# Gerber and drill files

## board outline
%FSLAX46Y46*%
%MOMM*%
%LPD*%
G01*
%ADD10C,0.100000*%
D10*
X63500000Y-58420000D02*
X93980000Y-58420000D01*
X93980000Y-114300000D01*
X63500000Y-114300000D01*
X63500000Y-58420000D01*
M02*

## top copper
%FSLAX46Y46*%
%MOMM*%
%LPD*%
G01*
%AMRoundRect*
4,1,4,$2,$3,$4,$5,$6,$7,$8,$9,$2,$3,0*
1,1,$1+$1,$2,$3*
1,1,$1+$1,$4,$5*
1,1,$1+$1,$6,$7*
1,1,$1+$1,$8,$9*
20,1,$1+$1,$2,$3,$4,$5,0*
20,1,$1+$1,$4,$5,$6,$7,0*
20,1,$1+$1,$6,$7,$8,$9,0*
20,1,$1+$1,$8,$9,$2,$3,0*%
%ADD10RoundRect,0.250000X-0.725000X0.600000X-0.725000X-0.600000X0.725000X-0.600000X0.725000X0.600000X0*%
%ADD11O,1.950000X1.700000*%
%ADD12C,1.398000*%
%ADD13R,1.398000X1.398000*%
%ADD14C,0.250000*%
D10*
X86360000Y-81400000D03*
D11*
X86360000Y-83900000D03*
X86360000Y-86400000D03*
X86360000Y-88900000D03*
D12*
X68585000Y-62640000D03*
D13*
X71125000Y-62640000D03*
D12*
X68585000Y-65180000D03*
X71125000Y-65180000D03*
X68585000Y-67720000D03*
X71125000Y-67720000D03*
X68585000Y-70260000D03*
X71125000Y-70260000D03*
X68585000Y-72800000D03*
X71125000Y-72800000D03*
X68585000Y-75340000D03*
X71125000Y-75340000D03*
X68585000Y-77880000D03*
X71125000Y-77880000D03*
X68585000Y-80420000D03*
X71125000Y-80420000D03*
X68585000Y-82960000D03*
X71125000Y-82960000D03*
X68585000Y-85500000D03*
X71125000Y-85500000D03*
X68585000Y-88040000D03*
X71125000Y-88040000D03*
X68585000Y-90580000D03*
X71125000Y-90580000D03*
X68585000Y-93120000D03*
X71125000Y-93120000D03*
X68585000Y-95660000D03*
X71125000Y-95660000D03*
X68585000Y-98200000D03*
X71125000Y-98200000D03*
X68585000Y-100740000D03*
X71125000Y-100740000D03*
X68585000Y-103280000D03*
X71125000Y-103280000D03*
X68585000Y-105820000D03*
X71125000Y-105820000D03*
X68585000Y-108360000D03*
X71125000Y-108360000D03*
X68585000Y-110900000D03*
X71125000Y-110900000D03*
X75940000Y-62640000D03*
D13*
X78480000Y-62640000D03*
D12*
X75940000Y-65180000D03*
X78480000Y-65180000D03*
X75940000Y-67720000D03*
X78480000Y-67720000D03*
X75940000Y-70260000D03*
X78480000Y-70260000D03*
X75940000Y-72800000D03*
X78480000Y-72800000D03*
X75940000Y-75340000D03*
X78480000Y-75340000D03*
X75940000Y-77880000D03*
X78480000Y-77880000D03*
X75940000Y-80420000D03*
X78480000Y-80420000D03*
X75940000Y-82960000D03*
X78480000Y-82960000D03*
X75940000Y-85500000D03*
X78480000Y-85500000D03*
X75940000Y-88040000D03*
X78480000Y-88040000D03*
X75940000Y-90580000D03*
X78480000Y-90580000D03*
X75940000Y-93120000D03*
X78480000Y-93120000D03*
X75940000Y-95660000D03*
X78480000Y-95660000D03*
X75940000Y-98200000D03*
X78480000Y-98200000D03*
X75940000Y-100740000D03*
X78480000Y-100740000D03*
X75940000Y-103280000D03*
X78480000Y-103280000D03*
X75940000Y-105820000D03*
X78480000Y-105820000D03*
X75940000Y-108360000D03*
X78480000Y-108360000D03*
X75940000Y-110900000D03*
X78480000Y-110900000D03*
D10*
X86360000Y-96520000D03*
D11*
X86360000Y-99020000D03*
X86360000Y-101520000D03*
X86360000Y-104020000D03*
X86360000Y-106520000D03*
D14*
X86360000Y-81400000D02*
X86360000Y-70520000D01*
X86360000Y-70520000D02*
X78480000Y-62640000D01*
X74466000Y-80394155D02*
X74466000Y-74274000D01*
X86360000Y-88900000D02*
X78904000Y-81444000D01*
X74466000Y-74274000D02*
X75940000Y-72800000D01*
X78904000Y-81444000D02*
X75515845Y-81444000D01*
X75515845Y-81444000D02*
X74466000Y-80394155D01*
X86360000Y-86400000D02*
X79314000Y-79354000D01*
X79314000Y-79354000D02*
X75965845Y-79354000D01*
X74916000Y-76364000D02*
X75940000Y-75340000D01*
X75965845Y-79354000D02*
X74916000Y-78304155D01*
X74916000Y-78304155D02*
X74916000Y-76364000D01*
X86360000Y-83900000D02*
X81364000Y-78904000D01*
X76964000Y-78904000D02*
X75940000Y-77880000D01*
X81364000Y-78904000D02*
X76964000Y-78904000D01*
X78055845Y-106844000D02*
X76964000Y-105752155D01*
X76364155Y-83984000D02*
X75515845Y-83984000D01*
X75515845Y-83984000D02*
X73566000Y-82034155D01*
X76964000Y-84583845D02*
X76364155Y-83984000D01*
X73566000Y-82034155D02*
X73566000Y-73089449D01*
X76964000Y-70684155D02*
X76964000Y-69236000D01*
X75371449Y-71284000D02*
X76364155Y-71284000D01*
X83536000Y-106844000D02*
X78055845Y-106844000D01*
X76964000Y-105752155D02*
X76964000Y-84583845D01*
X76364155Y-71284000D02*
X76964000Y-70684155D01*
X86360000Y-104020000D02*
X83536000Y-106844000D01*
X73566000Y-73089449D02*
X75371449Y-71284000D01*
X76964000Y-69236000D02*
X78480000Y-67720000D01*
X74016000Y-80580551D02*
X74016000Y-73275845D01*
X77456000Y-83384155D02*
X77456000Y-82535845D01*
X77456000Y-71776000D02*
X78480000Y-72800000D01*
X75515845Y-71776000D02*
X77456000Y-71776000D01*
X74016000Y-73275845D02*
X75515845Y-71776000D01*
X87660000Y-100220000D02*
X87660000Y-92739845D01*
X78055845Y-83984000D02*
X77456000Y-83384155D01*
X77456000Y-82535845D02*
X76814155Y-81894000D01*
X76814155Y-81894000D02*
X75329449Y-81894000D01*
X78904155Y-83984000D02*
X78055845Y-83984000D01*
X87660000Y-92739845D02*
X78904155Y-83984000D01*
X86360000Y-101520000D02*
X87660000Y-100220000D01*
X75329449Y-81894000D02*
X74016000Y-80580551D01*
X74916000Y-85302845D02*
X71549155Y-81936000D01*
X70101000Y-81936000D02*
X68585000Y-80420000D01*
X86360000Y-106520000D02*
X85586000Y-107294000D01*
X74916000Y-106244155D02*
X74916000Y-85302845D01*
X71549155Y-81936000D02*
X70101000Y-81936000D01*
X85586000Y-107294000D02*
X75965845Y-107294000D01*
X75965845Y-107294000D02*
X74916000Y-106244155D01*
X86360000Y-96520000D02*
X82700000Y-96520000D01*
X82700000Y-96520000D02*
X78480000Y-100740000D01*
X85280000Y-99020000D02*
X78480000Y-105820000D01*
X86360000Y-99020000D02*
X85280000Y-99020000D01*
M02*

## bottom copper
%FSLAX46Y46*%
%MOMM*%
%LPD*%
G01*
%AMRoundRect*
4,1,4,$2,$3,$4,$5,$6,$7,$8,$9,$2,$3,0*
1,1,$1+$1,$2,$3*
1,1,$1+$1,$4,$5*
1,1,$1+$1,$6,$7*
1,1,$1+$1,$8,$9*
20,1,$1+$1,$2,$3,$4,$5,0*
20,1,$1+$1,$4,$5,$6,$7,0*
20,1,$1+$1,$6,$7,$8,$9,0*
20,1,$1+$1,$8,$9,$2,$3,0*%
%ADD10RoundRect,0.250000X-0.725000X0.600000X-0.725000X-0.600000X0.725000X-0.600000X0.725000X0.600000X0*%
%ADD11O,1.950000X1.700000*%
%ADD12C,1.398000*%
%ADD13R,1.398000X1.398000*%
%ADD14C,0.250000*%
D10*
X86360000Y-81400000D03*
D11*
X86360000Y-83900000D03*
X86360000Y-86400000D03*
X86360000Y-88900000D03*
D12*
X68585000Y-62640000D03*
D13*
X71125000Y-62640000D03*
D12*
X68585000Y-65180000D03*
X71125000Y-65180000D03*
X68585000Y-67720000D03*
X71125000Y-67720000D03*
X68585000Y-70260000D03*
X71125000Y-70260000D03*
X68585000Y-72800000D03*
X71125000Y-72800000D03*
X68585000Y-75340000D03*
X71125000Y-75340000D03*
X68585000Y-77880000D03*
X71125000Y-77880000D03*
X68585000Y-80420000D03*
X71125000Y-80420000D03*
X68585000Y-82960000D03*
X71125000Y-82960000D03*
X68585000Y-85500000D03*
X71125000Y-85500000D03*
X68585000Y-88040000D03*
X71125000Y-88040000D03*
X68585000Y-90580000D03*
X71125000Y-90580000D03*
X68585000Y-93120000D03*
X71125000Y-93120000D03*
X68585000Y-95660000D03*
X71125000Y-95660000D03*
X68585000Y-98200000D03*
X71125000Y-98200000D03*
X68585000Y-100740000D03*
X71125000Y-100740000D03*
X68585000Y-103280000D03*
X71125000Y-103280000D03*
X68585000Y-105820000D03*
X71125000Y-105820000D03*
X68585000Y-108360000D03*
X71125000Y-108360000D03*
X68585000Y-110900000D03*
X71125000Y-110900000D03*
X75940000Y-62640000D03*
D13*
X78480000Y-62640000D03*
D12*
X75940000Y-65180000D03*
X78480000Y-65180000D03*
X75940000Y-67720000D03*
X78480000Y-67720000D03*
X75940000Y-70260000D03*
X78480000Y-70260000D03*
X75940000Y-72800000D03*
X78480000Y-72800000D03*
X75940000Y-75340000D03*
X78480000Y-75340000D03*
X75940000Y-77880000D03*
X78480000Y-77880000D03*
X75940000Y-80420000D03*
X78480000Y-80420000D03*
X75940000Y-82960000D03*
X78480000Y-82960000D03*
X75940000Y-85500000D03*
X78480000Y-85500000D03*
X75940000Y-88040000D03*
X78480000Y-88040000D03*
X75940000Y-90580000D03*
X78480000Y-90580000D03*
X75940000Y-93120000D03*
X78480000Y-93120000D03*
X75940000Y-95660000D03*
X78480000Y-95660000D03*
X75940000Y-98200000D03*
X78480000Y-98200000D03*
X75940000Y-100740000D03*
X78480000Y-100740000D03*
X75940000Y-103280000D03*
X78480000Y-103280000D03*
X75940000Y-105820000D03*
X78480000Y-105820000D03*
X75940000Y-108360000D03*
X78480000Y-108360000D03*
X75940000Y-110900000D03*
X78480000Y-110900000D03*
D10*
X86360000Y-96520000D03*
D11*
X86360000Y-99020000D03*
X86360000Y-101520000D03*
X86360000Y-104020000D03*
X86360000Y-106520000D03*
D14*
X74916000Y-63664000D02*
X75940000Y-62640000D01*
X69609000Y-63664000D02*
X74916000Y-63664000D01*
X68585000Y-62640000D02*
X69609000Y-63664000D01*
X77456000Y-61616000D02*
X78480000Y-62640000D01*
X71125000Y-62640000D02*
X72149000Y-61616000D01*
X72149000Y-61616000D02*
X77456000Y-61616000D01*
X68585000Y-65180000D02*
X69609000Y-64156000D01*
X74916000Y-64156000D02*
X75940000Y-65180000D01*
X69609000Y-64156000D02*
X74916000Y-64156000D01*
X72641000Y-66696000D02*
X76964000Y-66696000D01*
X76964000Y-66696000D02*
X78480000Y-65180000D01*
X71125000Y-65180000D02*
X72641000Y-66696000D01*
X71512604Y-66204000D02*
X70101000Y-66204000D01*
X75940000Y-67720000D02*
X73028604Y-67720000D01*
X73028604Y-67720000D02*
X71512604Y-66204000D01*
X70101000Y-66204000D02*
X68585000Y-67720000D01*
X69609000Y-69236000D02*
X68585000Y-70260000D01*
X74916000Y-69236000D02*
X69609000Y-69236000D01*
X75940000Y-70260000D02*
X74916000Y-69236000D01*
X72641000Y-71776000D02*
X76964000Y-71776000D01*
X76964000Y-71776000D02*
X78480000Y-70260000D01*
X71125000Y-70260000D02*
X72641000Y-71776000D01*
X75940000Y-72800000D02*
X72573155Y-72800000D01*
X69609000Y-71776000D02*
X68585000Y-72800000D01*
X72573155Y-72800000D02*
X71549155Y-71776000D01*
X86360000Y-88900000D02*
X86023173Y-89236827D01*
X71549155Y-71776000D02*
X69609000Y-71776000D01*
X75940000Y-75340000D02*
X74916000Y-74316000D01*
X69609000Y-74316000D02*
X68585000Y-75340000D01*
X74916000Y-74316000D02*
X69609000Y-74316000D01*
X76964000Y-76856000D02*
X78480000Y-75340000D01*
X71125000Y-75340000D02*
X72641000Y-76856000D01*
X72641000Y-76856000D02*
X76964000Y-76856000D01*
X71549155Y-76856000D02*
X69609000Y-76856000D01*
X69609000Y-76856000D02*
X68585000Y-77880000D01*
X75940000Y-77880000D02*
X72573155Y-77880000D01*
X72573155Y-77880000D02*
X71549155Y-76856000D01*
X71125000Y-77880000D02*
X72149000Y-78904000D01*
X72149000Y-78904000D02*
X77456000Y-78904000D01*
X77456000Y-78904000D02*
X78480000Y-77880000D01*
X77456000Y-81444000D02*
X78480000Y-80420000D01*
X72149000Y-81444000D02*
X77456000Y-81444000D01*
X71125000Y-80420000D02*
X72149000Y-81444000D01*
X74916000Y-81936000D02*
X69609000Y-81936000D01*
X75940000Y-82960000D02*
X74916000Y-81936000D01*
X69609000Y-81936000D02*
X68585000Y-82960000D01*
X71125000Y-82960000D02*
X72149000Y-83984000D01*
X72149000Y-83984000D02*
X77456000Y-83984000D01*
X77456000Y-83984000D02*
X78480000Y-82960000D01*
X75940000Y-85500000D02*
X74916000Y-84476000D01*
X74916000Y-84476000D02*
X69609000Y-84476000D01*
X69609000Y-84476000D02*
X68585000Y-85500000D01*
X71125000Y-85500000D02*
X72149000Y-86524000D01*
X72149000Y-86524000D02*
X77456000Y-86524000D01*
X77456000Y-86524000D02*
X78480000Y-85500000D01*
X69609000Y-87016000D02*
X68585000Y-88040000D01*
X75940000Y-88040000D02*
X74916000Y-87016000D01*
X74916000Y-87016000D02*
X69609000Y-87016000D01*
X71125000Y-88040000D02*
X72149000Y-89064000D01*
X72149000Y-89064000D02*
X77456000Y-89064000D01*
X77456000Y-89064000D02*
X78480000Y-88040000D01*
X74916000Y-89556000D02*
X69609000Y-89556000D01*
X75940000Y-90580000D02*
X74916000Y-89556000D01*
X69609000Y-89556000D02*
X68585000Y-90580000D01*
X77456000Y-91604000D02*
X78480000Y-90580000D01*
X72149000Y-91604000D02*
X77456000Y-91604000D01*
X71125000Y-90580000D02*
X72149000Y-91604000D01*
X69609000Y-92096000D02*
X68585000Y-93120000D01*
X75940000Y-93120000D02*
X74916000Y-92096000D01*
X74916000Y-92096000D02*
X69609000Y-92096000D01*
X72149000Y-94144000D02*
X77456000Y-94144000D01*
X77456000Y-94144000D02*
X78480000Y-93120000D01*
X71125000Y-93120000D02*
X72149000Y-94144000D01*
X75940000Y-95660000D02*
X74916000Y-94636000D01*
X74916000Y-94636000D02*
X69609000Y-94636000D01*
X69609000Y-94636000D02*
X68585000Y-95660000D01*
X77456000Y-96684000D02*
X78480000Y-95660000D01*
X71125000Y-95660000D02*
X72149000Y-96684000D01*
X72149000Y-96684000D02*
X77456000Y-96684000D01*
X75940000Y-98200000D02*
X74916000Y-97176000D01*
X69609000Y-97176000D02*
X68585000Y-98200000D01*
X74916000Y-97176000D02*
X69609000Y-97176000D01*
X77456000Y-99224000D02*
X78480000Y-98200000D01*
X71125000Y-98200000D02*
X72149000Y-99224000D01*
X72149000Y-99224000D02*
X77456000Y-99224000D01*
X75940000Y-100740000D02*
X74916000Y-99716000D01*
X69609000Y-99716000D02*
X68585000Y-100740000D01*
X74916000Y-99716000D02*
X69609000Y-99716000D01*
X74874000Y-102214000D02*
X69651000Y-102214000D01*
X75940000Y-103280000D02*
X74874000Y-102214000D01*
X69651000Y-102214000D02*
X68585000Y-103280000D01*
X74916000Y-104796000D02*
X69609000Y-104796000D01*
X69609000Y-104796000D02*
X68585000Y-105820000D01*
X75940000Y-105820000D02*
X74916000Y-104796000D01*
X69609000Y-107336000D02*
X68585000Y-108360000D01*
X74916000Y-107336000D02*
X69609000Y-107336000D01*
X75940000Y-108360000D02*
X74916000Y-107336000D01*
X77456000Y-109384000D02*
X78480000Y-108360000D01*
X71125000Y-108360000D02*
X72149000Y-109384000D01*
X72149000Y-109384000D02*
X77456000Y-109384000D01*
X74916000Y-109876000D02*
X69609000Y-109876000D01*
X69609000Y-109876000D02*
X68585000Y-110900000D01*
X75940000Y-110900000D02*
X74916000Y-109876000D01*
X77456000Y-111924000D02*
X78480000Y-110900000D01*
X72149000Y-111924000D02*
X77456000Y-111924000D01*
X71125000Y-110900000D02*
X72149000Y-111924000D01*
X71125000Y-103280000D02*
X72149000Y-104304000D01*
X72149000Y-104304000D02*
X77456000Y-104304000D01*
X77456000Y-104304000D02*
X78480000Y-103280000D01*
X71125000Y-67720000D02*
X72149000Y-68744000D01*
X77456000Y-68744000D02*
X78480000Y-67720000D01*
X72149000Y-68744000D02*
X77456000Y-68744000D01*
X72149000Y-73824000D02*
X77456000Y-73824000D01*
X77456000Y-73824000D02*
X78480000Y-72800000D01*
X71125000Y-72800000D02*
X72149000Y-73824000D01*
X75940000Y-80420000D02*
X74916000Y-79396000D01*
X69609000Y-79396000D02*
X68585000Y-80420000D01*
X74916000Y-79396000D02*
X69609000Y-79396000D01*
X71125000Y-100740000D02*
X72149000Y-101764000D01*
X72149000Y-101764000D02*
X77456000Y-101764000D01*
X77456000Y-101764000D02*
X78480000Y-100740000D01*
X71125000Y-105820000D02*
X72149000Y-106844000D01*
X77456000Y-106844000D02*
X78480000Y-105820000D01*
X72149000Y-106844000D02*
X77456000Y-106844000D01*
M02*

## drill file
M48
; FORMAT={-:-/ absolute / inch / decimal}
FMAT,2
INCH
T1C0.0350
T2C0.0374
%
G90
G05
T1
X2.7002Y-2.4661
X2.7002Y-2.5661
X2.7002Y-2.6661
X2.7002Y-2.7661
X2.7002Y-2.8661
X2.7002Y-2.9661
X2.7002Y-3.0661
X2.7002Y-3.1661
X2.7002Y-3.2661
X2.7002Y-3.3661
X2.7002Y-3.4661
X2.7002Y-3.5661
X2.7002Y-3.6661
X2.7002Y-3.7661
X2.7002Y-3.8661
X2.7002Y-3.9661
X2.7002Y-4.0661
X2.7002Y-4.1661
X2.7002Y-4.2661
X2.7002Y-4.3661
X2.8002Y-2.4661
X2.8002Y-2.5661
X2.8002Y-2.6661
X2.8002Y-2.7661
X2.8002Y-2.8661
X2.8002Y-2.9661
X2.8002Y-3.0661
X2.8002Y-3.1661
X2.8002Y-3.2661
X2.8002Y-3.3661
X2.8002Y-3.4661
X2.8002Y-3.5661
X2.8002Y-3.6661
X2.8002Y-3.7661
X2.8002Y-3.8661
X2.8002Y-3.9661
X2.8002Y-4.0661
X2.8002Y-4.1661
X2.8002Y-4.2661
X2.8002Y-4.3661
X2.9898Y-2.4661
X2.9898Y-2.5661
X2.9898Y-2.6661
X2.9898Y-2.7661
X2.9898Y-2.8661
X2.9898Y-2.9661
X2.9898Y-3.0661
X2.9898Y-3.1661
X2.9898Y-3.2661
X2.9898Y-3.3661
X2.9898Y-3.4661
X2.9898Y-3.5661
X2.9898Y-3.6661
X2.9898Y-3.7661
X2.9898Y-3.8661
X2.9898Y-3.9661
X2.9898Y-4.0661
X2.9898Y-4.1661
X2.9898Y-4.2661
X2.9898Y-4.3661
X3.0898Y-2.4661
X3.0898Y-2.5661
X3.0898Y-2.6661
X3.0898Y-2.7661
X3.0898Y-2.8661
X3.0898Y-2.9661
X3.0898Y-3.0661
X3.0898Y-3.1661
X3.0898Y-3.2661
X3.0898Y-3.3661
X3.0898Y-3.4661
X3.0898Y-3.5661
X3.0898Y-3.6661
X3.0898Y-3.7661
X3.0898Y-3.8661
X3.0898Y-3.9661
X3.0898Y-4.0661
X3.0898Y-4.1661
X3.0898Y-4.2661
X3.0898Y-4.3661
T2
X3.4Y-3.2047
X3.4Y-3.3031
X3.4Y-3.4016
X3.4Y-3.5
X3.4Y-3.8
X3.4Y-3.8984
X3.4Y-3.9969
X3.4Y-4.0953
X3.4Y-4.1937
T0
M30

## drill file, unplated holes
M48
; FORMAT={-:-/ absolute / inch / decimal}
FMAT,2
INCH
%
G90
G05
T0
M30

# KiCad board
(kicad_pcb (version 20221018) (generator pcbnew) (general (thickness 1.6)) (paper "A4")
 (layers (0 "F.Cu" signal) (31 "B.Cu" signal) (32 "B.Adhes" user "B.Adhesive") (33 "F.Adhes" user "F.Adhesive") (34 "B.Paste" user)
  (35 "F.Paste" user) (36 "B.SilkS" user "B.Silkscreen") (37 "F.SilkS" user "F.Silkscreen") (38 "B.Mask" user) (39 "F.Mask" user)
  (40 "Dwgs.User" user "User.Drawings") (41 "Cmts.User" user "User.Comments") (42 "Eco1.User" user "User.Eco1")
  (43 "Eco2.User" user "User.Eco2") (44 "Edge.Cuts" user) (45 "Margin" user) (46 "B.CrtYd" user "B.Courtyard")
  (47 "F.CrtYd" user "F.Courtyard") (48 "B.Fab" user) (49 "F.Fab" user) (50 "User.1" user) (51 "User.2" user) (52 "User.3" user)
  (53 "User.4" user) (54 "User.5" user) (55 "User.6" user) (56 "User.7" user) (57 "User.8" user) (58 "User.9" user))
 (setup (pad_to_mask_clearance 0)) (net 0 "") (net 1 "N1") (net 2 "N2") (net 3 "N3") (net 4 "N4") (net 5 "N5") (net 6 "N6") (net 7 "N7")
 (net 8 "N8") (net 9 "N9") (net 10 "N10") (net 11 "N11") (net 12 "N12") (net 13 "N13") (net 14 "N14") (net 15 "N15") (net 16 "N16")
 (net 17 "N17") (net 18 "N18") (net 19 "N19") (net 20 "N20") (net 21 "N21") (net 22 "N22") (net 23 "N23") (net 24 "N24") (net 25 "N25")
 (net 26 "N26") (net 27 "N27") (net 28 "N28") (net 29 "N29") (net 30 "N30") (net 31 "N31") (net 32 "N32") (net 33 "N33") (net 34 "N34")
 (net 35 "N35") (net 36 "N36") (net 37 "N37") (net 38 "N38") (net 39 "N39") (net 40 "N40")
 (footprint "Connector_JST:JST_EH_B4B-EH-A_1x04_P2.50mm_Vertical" (layer "F.Cu") (at 86.36 81.4 -90)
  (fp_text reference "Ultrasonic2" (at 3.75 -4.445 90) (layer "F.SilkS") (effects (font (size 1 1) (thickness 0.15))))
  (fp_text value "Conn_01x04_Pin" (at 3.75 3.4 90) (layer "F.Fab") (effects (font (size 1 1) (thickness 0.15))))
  (pad "1" thru_hole roundrect (at 0 0 270) (size 1.7 1.95) (drill 0.95) (layers "*.Cu" "*.Mask") (roundrect_rratio 0.1470588235)
   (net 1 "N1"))
  (pad "2" thru_hole oval (at 2.5 0 270) (size 1.7 1.95) (drill 0.95) (layers "*.Cu" "*.Mask") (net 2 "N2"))
  (pad "3" thru_hole oval (at 5 0 270) (size 1.7 1.95) (drill 0.95) (layers "*.Cu" "*.Mask") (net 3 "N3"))
  (pad "4" thru_hole oval (at 7.5 0 270) (size 1.7 1.95) (drill 0.95) (layers "*.Cu" "*.Mask") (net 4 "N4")))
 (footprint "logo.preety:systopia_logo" (layer "F.Cu") (at 87.63 68.58)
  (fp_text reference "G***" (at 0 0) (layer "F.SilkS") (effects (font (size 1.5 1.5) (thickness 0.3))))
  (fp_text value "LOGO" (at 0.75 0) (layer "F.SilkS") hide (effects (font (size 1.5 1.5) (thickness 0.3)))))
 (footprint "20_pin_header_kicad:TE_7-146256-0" (layer "F.Cu") (at 69.855 86.77 -90)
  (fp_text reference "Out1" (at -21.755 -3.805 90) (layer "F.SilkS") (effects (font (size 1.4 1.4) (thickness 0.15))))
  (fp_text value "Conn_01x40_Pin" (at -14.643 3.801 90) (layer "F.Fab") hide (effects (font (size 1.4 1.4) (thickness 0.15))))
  (pad "1" thru_hole circle (at -24.13 1.27 270) (size 1.398 1.398) (drill 0.89) (layers "*.Cu" "*.Mask") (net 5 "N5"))
  (pad "2" thru_hole rect (at -24.13 -1.27 270) (size 1.398 1.398) (drill 0.89) (layers "*.Cu" "*.Mask") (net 1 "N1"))
  (pad "3" thru_hole circle (at -21.59 1.27 270) (size 1.398 1.398) (drill 0.89) (layers "*.Cu" "*.Mask") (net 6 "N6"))
  (pad "4" thru_hole circle (at -21.59 -1.27 270) (size 1.398 1.398) (drill 0.89) (layers "*.Cu" "*.Mask") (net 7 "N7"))
  (pad "5" thru_hole circle (at -19.05 1.27 270) (size 1.398 1.398) (drill 0.89) (layers "*.Cu" "*.Mask") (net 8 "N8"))
  (pad "6" thru_hole circle (at -19.05 -1.27 270) (size 1.398 1.398) (drill 0.89) (layers "*.Cu" "*.Mask") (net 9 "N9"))
  (pad "7" thru_hole circle (at -16.51 1.27 270) (size 1.398 1.398) (drill 0.89) (layers "*.Cu" "*.Mask") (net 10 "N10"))
  (pad "8" thru_hole circle (at -16.51 -1.27 270) (size 1.398 1.398) (drill 0.89) (layers "*.Cu" "*.Mask") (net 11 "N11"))
  (pad "9" thru_hole circle (at -13.97 1.27 270) (size 1.398 1.398) (drill 0.89) (layers "*.Cu" "*.Mask") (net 4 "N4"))
  (pad "10" thru_hole circle (at -13.97 -1.27 270) (size 1.398 1.398) (drill 0.89) (layers "*.Cu" "*.Mask") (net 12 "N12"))
  (pad "11" thru_hole circle (at -11.43 1.27 270) (size 1.398 1.398) (drill 0.89) (layers "*.Cu" "*.Mask") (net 3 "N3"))
  (pad "12" thru_hole circle (at -11.43 -1.27 270) (size 1.398 1.398) (drill 0.89) (layers "*.Cu" "*.Mask") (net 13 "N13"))
  (pad "13" thru_hole circle (at -8.89 1.27 270) (size 1.398 1.398) (drill 0.89) (layers "*.Cu" "*.Mask") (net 2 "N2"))
  (pad "14" thru_hole circle (at -8.89 -1.27 270) (size 1.398 1.398) (drill 0.89) (layers "*.Cu" "*.Mask") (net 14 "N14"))
  (pad "15" thru_hole circle (at -6.35 1.27 270) (size 1.398 1.398) (drill 0.89) (layers "*.Cu" "*.Mask") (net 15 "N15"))
  (pad "16" thru_hole circle (at -6.35 -1.27 270) (size 1.398 1.398) (drill 0.89) (layers "*.Cu" "*.Mask") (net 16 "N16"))
  (pad "17" thru_hole circle (at -3.81 1.27 270) (size 1.398 1.398) (drill 0.89) (layers "*.Cu" "*.Mask") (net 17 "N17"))
  (pad "18" thru_hole circle (at -3.81 -1.27 270) (size 1.398 1.398) (drill 0.89) (layers "*.Cu" "*.Mask") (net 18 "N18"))
  (pad "19" thru_hole circle (at -1.27 1.27 270) (size 1.398 1.398) (drill 0.89) (layers "*.Cu" "*.Mask") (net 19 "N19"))
  (pad "20" thru_hole circle (at -1.27 -1.27 270) (size 1.398 1.398) (drill 0.89) (layers "*.Cu" "*.Mask") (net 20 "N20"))
  (pad "21" thru_hole circle (at 1.27 1.27 270) (size 1.398 1.398) (drill 0.89) (layers "*.Cu" "*.Mask") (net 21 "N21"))
  (pad "22" thru_hole circle (at 1.27 -1.27 270) (size 1.398 1.398) (drill 0.89) (layers "*.Cu" "*.Mask") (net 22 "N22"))
  (pad "23" thru_hole circle (at 3.81 1.27 270) (size 1.398 1.398) (drill 0.89) (layers "*.Cu" "*.Mask") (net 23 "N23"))
  (pad "24" thru_hole circle (at 3.81 -1.27 270) (size 1.398 1.398) (drill 0.89) (layers "*.Cu" "*.Mask") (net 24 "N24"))
  (pad "25" thru_hole circle (at 6.35 1.27 270) (size 1.398 1.398) (drill 0.89) (layers "*.Cu" "*.Mask") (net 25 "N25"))
  (pad "26" thru_hole circle (at 6.35 -1.27 270) (size 1.398 1.398) (drill 0.89) (layers "*.Cu" "*.Mask") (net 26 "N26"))
  (pad "27" thru_hole circle (at 8.89 1.27 270) (size 1.398 1.398) (drill 0.89) (layers "*.Cu" "*.Mask") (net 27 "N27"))
  (pad "28" thru_hole circle (at 8.89 -1.27 270) (size 1.398 1.398) (drill 0.89) (layers "*.Cu" "*.Mask") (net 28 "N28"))
  (pad "29" thru_hole circle (at 11.43 1.27 270) (size 1.398 1.398) (drill 0.89) (layers "*.Cu" "*.Mask") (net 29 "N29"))
  (pad "30" thru_hole circle (at 11.43 -1.27 270) (size 1.398 1.398) (drill 0.89) (layers "*.Cu" "*.Mask") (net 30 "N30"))
  (pad "31" thru_hole circle (at 13.97 1.27 270) (size 1.398 1.398) (drill 0.89) (layers "*.Cu" "*.Mask") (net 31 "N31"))
  (pad "32" thru_hole circle (at 13.97 -1.27 270) (size 1.398 1.398) (drill 0.89) (layers "*.Cu" "*.Mask") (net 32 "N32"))
  (pad "33" thru_hole circle (at 16.51 1.27 270) (size 1.398 1.398) (drill 0.89) (layers "*.Cu" "*.Mask") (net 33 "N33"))
  (pad "34" thru_hole circle (at 16.51 -1.27 270) (size 1.398 1.398) (drill 0.89) (layers "*.Cu" "*.Mask") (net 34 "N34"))
  (pad "35" thru_hole circle (at 19.05 1.27 270) (size 1.398 1.398) (drill 0.89) (layers "*.Cu" "*.Mask") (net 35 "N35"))
  (pad "36" thru_hole circle (at 19.05 -1.27 270) (size 1.398 1.398) (drill 0.89) (layers "*.Cu" "*.Mask") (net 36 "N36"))
  (pad "37" thru_hole circle (at 21.59 1.27 270) (size 1.398 1.398) (drill 0.89) (layers "*.Cu" "*.Mask") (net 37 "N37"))
  (pad "38" thru_hole circle (at 21.59 -1.27 270) (size 1.398 1.398) (drill 0.89) (layers "*.Cu" "*.Mask") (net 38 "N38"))
  (pad "39" thru_hole circle (at 24.13 1.27 270) (size 1.398 1.398) (drill 0.89) (layers "*.Cu" "*.Mask") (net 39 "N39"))
  (pad "40" thru_hole circle (at 24.13 -1.27 270) (size 1.398 1.398) (drill 0.89) (layers "*.Cu" "*.Mask") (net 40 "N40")))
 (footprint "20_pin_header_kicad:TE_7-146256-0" (layer "F.Cu") (at 77.21 86.77 -90)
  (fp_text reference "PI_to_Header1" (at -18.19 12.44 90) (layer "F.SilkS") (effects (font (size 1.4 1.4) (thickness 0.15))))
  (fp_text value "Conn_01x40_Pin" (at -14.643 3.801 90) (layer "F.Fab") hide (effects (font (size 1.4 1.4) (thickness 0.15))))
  (pad "1" thru_hole circle (at -24.13 1.27 270) (size 1.398 1.398) (drill 0.89) (layers "*.Cu" "*.Mask") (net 5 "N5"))
  (pad "2" thru_hole rect (at -24.13 -1.27 270) (size 1.398 1.398) (drill 0.89) (layers "*.Cu" "*.Mask") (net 1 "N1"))
  (pad "3" thru_hole circle (at -21.59 1.27 270) (size 1.398 1.398) (drill 0.89) (layers "*.Cu" "*.Mask") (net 6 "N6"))
  (pad "4" thru_hole circle (at -21.59 -1.27 270) (size 1.398 1.398) (drill 0.89) (layers "*.Cu" "*.Mask") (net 7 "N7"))
  (pad "5" thru_hole circle (at -19.05 1.27 270) (size 1.398 1.398) (drill 0.89) (layers "*.Cu" "*.Mask") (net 8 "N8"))
  (pad "6" thru_hole circle (at -19.05 -1.27 270) (size 1.398 1.398) (drill 0.89) (layers "*.Cu" "*.Mask") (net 9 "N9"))
  (pad "7" thru_hole circle (at -16.51 1.27 270) (size 1.398 1.398) (drill 0.89) (layers "*.Cu" "*.Mask") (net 10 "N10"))
  (pad "8" thru_hole circle (at -16.51 -1.27 270) (size 1.398 1.398) (drill 0.89) (layers "*.Cu" "*.Mask") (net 11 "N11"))
  (pad "9" thru_hole circle (at -13.97 1.27 270) (size 1.398 1.398) (drill 0.89) (layers "*.Cu" "*.Mask") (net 4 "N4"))
  (pad "10" thru_hole circle (at -13.97 -1.27 270) (size 1.398 1.398) (drill 0.89) (layers "*.Cu" "*.Mask") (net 12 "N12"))
  (pad "11" thru_hole circle (at -11.43 1.27 270) (size 1.398 1.398) (drill 0.89) (layers "*.Cu" "*.Mask") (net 3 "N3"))
  (pad "12" thru_hole circle (at -11.43 -1.27 270) (size 1.398 1.398) (drill 0.89) (layers "*.Cu" "*.Mask") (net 13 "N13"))
  (pad "13" thru_hole circle (at -8.89 1.27 270) (size 1.398 1.398) (drill 0.89) (layers "*.Cu" "*.Mask") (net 2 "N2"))
  (pad "14" thru_hole circle (at -8.89 -1.27 270) (size 1.398 1.398) (drill 0.89) (layers "*.Cu" "*.Mask") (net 14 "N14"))
  (pad "15" thru_hole circle (at -6.35 1.27 270) (size 1.398 1.398) (drill 0.89) (layers "*.Cu" "*.Mask") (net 15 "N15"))
  (pad "16" thru_hole circle (at -6.35 -1.27 270) (size 1.398 1.398) (drill 0.89) (layers "*.Cu" "*.Mask") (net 16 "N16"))
  (pad "17" thru_hole circle (at -3.81 1.27 270) (size 1.398 1.398) (drill 0.89) (layers "*.Cu" "*.Mask") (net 17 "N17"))
  (pad "18" thru_hole circle (at -3.81 -1.27 270) (size 1.398 1.398) (drill 0.89) (layers "*.Cu" "*.Mask") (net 18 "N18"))
  (pad "19" thru_hole circle (at -1.27 1.27 270) (size 1.398 1.398) (drill 0.89) (layers "*.Cu" "*.Mask") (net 19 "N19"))
  (pad "20" thru_hole circle (at -1.27 -1.27 270) (size 1.398 1.398) (drill 0.89) (layers "*.Cu" "*.Mask") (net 20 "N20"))
  (pad "21" thru_hole circle (at 1.27 1.27 270) (size 1.398 1.398) (drill 0.89) (layers "*.Cu" "*.Mask") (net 21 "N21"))
  (pad "22" thru_hole circle (at 1.27 -1.27 270) (size 1.398 1.398) (drill 0.89) (layers "*.Cu" "*.Mask") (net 22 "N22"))
  (pad "23" thru_hole circle (at 3.81 1.27 270) (size 1.398 1.398) (drill 0.89) (layers "*.Cu" "*.Mask") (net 23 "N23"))
  (pad "24" thru_hole circle (at 3.81 -1.27 270) (size 1.398 1.398) (drill 0.89) (layers "*.Cu" "*.Mask") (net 24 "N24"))
  (pad "25" thru_hole circle (at 6.35 1.27 270) (size 1.398 1.398) (drill 0.89) (layers "*.Cu" "*.Mask") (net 25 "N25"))
  (pad "26" thru_hole circle (at 6.35 -1.27 270) (size 1.398 1.398) (drill 0.89) (layers "*.Cu" "*.Mask") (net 26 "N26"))
  (pad "27" thru_hole circle (at 8.89 1.27 270) (size 1.398 1.398) (drill 0.89) (layers "*.Cu" "*.Mask") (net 27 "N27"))
  (pad "28" thru_hole circle (at 8.89 -1.27 270) (size 1.398 1.398) (drill 0.89) (layers "*.Cu" "*.Mask") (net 28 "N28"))
  (pad "29" thru_hole circle (at 11.43 1.27 270) (size 1.398 1.398) (drill 0.89) (layers "*.Cu" "*.Mask") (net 29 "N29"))
  (pad "30" thru_hole circle (at 11.43 -1.27 270) (size 1.398 1.398) (drill 0.89) (layers "*.Cu" "*.Mask") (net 30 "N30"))
  (pad "31" thru_hole circle (at 13.97 1.27 270) (size 1.398 1.398) (drill 0.89) (layers "*.Cu" "*.Mask") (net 31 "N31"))
  (pad "32" thru_hole circle (at 13.97 -1.27 270) (size 1.398 1.398) (drill 0.89) (layers "*.Cu" "*.Mask") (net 32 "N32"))
  (pad "33" thru_hole circle (at 16.51 1.27 270) (size 1.398 1.398) (drill 0.89) (layers "*.Cu" "*.Mask") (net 33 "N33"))
  (pad "34" thru_hole circle (at 16.51 -1.27 270) (size 1.398 1.398) (drill 0.89) (layers "*.Cu" "*.Mask") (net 34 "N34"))
  (pad "35" thru_hole circle (at 19.05 1.27 270) (size 1.398 1.398) (drill 0.89) (layers "*.Cu" "*.Mask") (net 35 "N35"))
  (pad "36" thru_hole circle (at 19.05 -1.27 270) (size 1.398 1.398) (drill 0.89) (layers "*.Cu" "*.Mask") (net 36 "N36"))
  (pad "37" thru_hole circle (at 21.59 1.27 270) (size 1.398 1.398) (drill 0.89) (layers "*.Cu" "*.Mask") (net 37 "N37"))
  (pad "38" thru_hole circle (at 21.59 -1.27 270) (size 1.398 1.398) (drill 0.89) (layers "*.Cu" "*.Mask") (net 38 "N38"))
  (pad "39" thru_hole circle (at 24.13 1.27 270) (size 1.398 1.398) (drill 0.89) (layers "*.Cu" "*.Mask") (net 39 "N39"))
  (pad "40" thru_hole circle (at 24.13 -1.27 270) (size 1.398 1.398) (drill 0.89) (layers "*.Cu" "*.Mask") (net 40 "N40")))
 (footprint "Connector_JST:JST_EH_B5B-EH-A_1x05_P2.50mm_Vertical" (layer "F.Cu") (at 86.36 96.52 -90)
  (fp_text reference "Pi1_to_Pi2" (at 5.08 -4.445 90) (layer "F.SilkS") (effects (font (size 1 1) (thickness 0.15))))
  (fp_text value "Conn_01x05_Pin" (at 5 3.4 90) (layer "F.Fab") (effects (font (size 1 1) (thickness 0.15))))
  (pad "1" thru_hole roundrect (at 0 0 270) (size 1.7 1.95) (drill 0.95) (layers "*.Cu" "*.Mask") (roundrect_rratio 0.1470588235)
   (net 32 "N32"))
  (pad "2" thru_hole oval (at 2.5 0 270) (size 1.7 1.95) (drill 0.95) (layers "*.Cu" "*.Mask") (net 36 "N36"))
  (pad "3" thru_hole oval (at 5 0 270) (size 1.7 1.95) (drill 0.95) (layers "*.Cu" "*.Mask") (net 12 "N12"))
  (pad "4" thru_hole oval (at 7.5 0 270) (size 1.7 1.95) (drill 0.95) (layers "*.Cu" "*.Mask") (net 9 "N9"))
  (pad "5" thru_hole oval (at 10 0 270) (size 1.7 1.95) (drill 0.95) (layers "*.Cu" "*.Mask") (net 15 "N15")))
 (gr_rect (start 63.5 58.42) (end 93.98 114.3) (stroke (width 0.1) (type default)) (fill none) (layer "Edge.Cuts"))
 (segment (start 74.916 63.664) (end 75.94 62.64) (width 0.25) (layer "B.Cu") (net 5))
 (segment (start 69.609 63.664) (end 74.916 63.664) (width 0.25) (layer "B.Cu") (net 5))
 (segment (start 68.585 62.64) (end 69.609 63.664) (width 0.25) (layer "B.Cu") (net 5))
 (segment (start 86.36 81.4) (end 86.36 70.52) (width 0.25) (layer "F.Cu") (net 1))
 (segment (start 86.36 70.52) (end 78.48 62.64) (width 0.25) (layer "F.Cu") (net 1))
 (segment (start 77.456 61.616) (end 78.48 62.64) (width 0.25) (layer "B.Cu") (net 1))
 (segment (start 71.125 62.64) (end 72.149 61.616) (width 0.25) (layer "B.Cu") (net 1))
 (segment (start 72.149 61.616) (end 77.456 61.616) (width 0.25) (layer "B.Cu") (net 1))
 (segment (start 68.585 65.18) (end 69.609 64.156) (width 0.25) (layer "B.Cu") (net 6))
 (segment (start 74.916 64.156) (end 75.94 65.18) (width 0.25) (layer "B.Cu") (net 6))
 (segment (start 69.609 64.156) (end 74.916 64.156) (width 0.25) (layer "B.Cu") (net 6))
 (segment (start 72.641 66.696) (end 76.964 66.696) (width 0.25) (layer "B.Cu") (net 7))
 (segment (start 76.964 66.696) (end 78.48 65.18) (width 0.25) (layer "B.Cu") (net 7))
 (segment (start 71.125 65.18) (end 72.641 66.696) (width 0.25) (layer "B.Cu") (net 7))
 (segment (start 71.512604 66.204) (end 70.101 66.204) (width 0.25) (layer "B.Cu") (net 8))
 (segment (start 75.94 67.72) (end 73.028604 67.72) (width 0.25) (layer "B.Cu") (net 8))
 (segment (start 73.028604 67.72) (end 71.512604 66.204) (width 0.25) (layer "B.Cu") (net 8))
 (segment (start 70.101 66.204) (end 68.585 67.72) (width 0.25) (layer "B.Cu") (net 8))
 (segment (start 69.609 69.236) (end 68.585 70.26) (width 0.25) (layer "B.Cu") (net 10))
 (segment (start 74.916 69.236) (end 69.609 69.236) (width 0.25) (layer "B.Cu") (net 10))
 (segment (start 75.94 70.26) (end 74.916 69.236) (width 0.25) (layer "B.Cu") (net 10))
 (segment (start 72.641 71.776) (end 76.964 71.776) (width 0.25) (layer "B.Cu") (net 11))
 (segment (start 76.964 71.776) (end 78.48 70.26) (width 0.25) (layer "B.Cu") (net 11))
 (segment (start 71.125 70.26) (end 72.641 71.776) (width 0.25) (layer "B.Cu") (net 11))
 (segment (start 74.466 80.394155) (end 74.466 74.274) (width 0.25) (layer "F.Cu") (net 4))
 (segment (start 86.36 88.9) (end 78.904 81.444) (width 0.25) (layer "F.Cu") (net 4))
 (segment (start 74.466 74.274) (end 75.94 72.8) (width 0.25) (layer "F.Cu") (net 4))
 (segment (start 78.904 81.444) (end 75.515845 81.444) (width 0.25) (layer "F.Cu") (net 4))
 (segment (start 75.515845 81.444) (end 74.466 80.394155) (width 0.25) (layer "F.Cu") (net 4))
 (segment (start 75.94 72.8) (end 72.573155 72.8) (width 0.25) (layer "B.Cu") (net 4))
 (segment (start 69.609 71.776) (end 68.585 72.8) (width 0.25) (layer "B.Cu") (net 4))
 (segment (start 72.573155 72.8) (end 71.549155 71.776) (width 0.25) (layer "B.Cu") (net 4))
 (segment (start 86.36 88.9) (end 86.023173 89.236827) (width 0.25) (layer "B.Cu") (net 4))
 (segment (start 71.549155 71.776) (end 69.609 71.776) (width 0.25) (layer "B.Cu") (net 4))
 (segment (start 86.36 86.4) (end 79.314 79.354) (width 0.25) (layer "F.Cu") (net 3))
 (segment (start 79.314 79.354) (end 75.965845 79.354) (width 0.25) (layer "F.Cu") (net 3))
 (segment (start 74.916 76.364) (end 75.94 75.34) (width 0.25) (layer "F.Cu") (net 3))
 (segment (start 75.965845 79.354) (end 74.916 78.304155) (width 0.25) (layer "F.Cu") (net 3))
 (segment (start 74.916 78.304155) (end 74.916 76.364) (width 0.25) (layer "F.Cu") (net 3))
 (segment (start 75.94 75.34) (end 74.916 74.316) (width 0.25) (layer "B.Cu") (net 3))
 (segment (start 69.609 74.316) (end 68.585 75.34) (width 0.25) (layer "B.Cu") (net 3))
 (segment (start 74.916 74.316) (end 69.609 74.316) (width 0.25) (layer "B.Cu") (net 3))
 (segment (start 76.964 76.856) (end 78.48 75.34) (width 0.25) (layer "B.Cu") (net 13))
 (segment (start 71.125 75.34) (end 72.641 76.856) (width 0.25) (layer "B.Cu") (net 13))
 (segment (start 72.641 76.856) (end 76.964 76.856) (width 0.25) (layer "B.Cu") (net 13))
 (segment (start 86.36 83.9) (end 81.364 78.904) (width 0.25) (layer "F.Cu") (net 2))
 (segment (start 76.964 78.904) (end 75.94 77.88) (width 0.25) (layer "F.Cu") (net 2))
 (segment (start 81.364 78.904) (end 76.964 78.904) (width 0.25) (layer "F.Cu") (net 2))
 (segment (start 71.549155 76.856) (end 69.609 76.856) (width 0.25) (layer "B.Cu") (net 2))
 (segment (start 69.609 76.856) (end 68.585 77.88) (width 0.25) (layer "B.Cu") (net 2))
 (segment (start 75.94 77.88) (end 72.573155 77.88) (width 0.25) (layer "B.Cu") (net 2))
 (segment (start 72.573155 77.88) (end 71.549155 76.856) (width 0.25) (layer "B.Cu") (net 2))
 (segment (start 71.125 77.88) (end 72.149 78.904) (width 0.25) (layer "B.Cu") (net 14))
 (segment (start 72.149 78.904) (end 77.456 78.904) (width 0.25) (layer "B.Cu") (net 14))
 (segment (start 77.456 78.904) (end 78.48 77.88) (width 0.25) (layer "B.Cu") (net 14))
 (segment (start 77.456 81.444) (end 78.48 80.42) (width 0.25) (layer "B.Cu") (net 16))
 (segment (start 72.149 81.444) (end 77.456 81.444) (width 0.25) (layer "B.Cu") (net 16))
 (segment (start 71.125 80.42) (end 72.149 81.444) (width 0.25) (layer "B.Cu") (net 16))
 (segment (start 74.916 81.936) (end 69.609 81.936) (width 0.25) (layer "B.Cu") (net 17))
 (segment (start 75.94 82.96) (end 74.916 81.936) (width 0.25) (layer "B.Cu") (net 17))
 (segment (start 69.609 81.936) (end 68.585 82.96) (width 0.25) (layer "B.Cu") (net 17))
 (segment (start 71.125 82.96) (end 72.149 83.984) (width 0.25) (layer "B.Cu") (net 18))
 (segment (start 72.149 83.984) (end 77.456 83.984) (width 0.25) (layer "B.Cu") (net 18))
 (segment (start 77.456 83.984) (end 78.48 82.96) (width 0.25) (layer "B.Cu") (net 18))
 (segment (start 75.94 85.5) (end 74.916 84.476) (width 0.25) (layer "B.Cu") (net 19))
 (segment (start 74.916 84.476) (end 69.609 84.476) (width 0.25) (layer "B.Cu") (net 19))
 (segment (start 69.609 84.476) (end 68.585 85.5) (width 0.25) (layer "B.Cu") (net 19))
 (segment (start 71.125 85.5) (end 72.149 86.524) (width 0.25) (layer "B.Cu") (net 20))
 (segment (start 72.149 86.524) (end 77.456 86.524) (width 0.25) (layer "B.Cu") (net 20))
 (segment (start 77.456 86.524) (end 78.48 85.5) (width 0.25) (layer "B.Cu") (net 20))
 (segment (start 69.609 87.016) (end 68.585 88.04) (width 0.25) (layer "B.Cu") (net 21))
 (segment (start 75.94 88.04) (end 74.916 87.016) (width 0.25) (layer "B.Cu") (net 21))
 (segment (start 74.916 87.016) (end 69.609 87.016) (width 0.25) (layer "B.Cu") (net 21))
 (segment (start 71.125 88.04) (end 72.149 89.064) (width 0.25) (layer "B.Cu") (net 22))
 (segment (start 72.149 89.064) (end 77.456 89.064) (width 0.25) (layer "B.Cu") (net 22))
 (segment (start 77.456 89.064) (end 78.48 88.04) (width 0.25) (layer "B.Cu") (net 22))
 (segment (start 74.916 89.556) (end 69.609 89.556) (width 0.25) (layer "B.Cu") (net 23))
 (segment (start 75.94 90.58) (end 74.916 89.556) (width 0.25) (layer "B.Cu") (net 23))
 (segment (start 69.609 89.556) (end 68.585 90.58) (width 0.25) (layer "B.Cu") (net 23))
 (segment (start 77.456 91.604) (end 78.48 90.58) (width 0.25) (layer "B.Cu") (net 24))
 (segment (start 72.149 91.604) (end 77.456 91.604) (width 0.25) (layer "B.Cu") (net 24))
 (segment (start 71.125 90.58) (end 72.149 91.604) (width 0.25) (layer "B.Cu") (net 24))
 (segment (start 69.609 92.096) (end 68.585 93.12) (width 0.25) (layer "B.Cu") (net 25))
 (segment (start 75.94 93.12) (end 74.916 92.096) (width 0.25) (layer "B.Cu") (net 25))
 (segment (start 74.916 92.096) (end 69.609 92.096) (width 0.25) (layer "B.Cu") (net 25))
 (segment (start 72.149 94.144) (end 77.456 94.144) (width 0.25) (layer "B.Cu") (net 26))
 (segment (start 77.456 94.144) (end 78.48 93.12) (width 0.25) (layer "B.Cu") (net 26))
 (segment (start 71.125 93.12) (end 72.149 94.144) (width 0.25) (layer "B.Cu") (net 26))
 (segment (start 75.94 95.66) (end 74.916 94.636) (width 0.25) (layer "B.Cu") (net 27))
 (segment (start 74.916 94.636) (end 69.609 94.636) (width 0.25) (layer "B.Cu") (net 27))
 (segment (start 69.609 94.636) (end 68.585 95.66) (width 0.25) (layer "B.Cu") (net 27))
 (segment (start 77.456 96.684) (end 78.48 95.66) (width 0.25) (layer "B.Cu") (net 28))
 (segment (start 71.125 95.66) (end 72.149 96.684) (width 0.25) (layer "B.Cu") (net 28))
 (segment (start 72.149 96.684) (end 77.456 96.684) (width 0.25) (layer "B.Cu") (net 28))
 (segment (start 75.94 98.2) (end 74.916 97.176) (width 0.25) (layer "B.Cu") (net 29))
 (segment (start 69.609 97.176) (end 68.585 98.2) (width 0.25) (layer "B.Cu") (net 29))
 (segment (start 74.916 97.176) (end 69.609 97.176) (width 0.25) (layer "B.Cu") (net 29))
 (segment (start 77.456 99.224) (end 78.48 98.2) (width 0.25) (layer "B.Cu") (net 30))
 (segment (start 71.125 98.2) (end 72.149 99.224) (width 0.25) (layer "B.Cu") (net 30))
 (segment (start 72.149 99.224) (end 77.456 99.224) (width 0.25) (layer "B.Cu") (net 30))
 (segment (start 75.94 100.74) (end 74.916 99.716) (width 0.25) (layer "B.Cu") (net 31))
 (segment (start 69.609 99.716) (end 68.585 100.74) (width 0.25) (layer "B.Cu") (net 31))
 (segment (start 74.916 99.716) (end 69.609 99.716) (width 0.25) (layer "B.Cu") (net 31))
 (segment (start 74.874 102.214) (end 69.651 102.214) (width 0.25) (layer "B.Cu") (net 33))
 (segment (start 75.94 103.28) (end 74.874 102.214) (width 0.25) (layer "B.Cu") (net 33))
 (segment (start 69.651 102.214) (end 68.585 103.28) (width 0.25) (layer "B.Cu") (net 33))
 (segment (start 74.916 104.796) (end 69.609 104.796) (width 0.25) (layer "B.Cu") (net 35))
 (segment (start 69.609 104.796) (end 68.585 105.82) (width 0.25) (layer "B.Cu") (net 35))
 (segment (start 75.94 105.82) (end 74.916 104.796) (width 0.25) (layer "B.Cu") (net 35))
 (segment (start 69.609 107.336) (end 68.585 108.36) (width 0.25) (layer "B.Cu") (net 37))
 (segment (start 74.916 107.336) (end 69.609 107.336) (width 0.25) (layer "B.Cu") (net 37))
 (segment (start 75.94 108.36) (end 74.916 107.336) (width 0.25) (layer "B.Cu") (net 37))
 (segment (start 77.456 109.384) (end 78.48 108.36) (width 0.25) (layer "B.Cu") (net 38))
 (segment (start 71.125 108.36) (end 72.149 109.384) (width 0.25) (layer "B.Cu") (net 38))
 (segment (start 72.149 109.384) (end 77.456 109.384) (width 0.25) (layer "B.Cu") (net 38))
 (segment (start 74.916 109.876) (end 69.609 109.876) (width 0.25) (layer "B.Cu") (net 39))
 (segment (start 69.609 109.876) (end 68.585 110.9) (width 0.25) (layer "B.Cu") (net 39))
 (segment (start 75.94 110.9) (end 74.916 109.876) (width 0.25) (layer "B.Cu") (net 39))
 (segment (start 77.456 111.924) (end 78.48 110.9) (width 0.25) (layer "B.Cu") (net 40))
 (segment (start 72.149 111.924) (end 77.456 111.924) (width 0.25) (layer "B.Cu") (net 40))
 (segment (start 71.125 110.9) (end 72.149 111.924) (width 0.25) (layer "B.Cu") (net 40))
 (segment (start 71.125 103.28) (end 72.149 104.304) (width 0.25) (layer "B.Cu") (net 34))
 (segment (start 72.149 104.304) (end 77.456 104.304) (width 0.25) (layer "B.Cu") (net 34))
 (segment (start 77.456 104.304) (end 78.48 103.28) (width 0.25) (layer "B.Cu") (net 34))
 (segment (start 78.055845 106.844) (end 76.964 105.752155) (width 0.25) (layer "F.Cu") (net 9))
 (segment (start 76.364155 83.984) (end 75.515845 83.984) (width 0.25) (layer "F.Cu") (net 9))
 (segment (start 75.515845 83.984) (end 73.566 82.034155) (width 0.25) (layer "F.Cu") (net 9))
 (segment (start 76.964 84.583845) (end 76.364155 83.984) (width 0.25) (layer "F.Cu") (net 9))
 (segment (start 73.566 82.034155) (end 73.566 73.089449) (width 0.25) (layer "F.Cu") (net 9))
 (segment (start 76.964 70.684155) (end 76.964 69.236) (width 0.25) (layer "F.Cu") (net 9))
 (segment (start 75.371449 71.284) (end 76.364155 71.284) (width 0.25) (layer "F.Cu") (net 9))
 (segment (start 83.536 106.844) (end 78.055845 106.844) (width 0.25) (layer "F.Cu") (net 9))
 (segment (start 76.964 105.752155) (end 76.964 84.583845) (width 0.25) (layer "F.Cu") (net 9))
 (segment (start 76.364155 71.284) (end 76.964 70.684155) (width 0.25) (layer "F.Cu") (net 9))
 (segment (start 86.36 104.02) (end 83.536 106.844) (width 0.25) (layer "F.Cu") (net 9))
 (segment (start 73.566 73.089449) (end 75.371449 71.284) (width 0.25) (layer "F.Cu") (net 9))
 (segment (start 76.964 69.236) (end 78.48 67.72) (width 0.25) (layer "F.Cu") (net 9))
 (segment (start 71.125 67.72) (end 72.149 68.744) (width 0.25) (layer "B.Cu") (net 9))
 (segment (start 77.456 68.744) (end 78.48 67.72) (width 0.25) (layer "B.Cu") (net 9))
 (segment (start 72.149 68.744) (end 77.456 68.744) (width 0.25) (layer "B.Cu") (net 9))
 (segment (start 74.016 80.580551) (end 74.016 73.275845) (width 0.25) (layer "F.Cu") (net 12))
 (segment (start 77.456 83.384155) (end 77.456 82.535845) (width 0.25) (layer "F.Cu") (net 12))
 (segment (start 77.456 71.776) (end 78.48 72.8) (width 0.25) (layer "F.Cu") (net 12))
 (segment (start 75.515845 71.776) (end 77.456 71.776) (width 0.25) (layer "F.Cu") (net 12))
 (segment (start 74.016 73.275845) (end 75.515845 71.776) (width 0.25) (layer "F.Cu") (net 12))
 (segment (start 87.66 100.22) (end 87.66 92.739845) (width 0.25) (layer "F.Cu") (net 12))
 (segment (start 78.055845 83.984) (end 77.456 83.384155) (width 0.25) (layer "F.Cu") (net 12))
 (segment (start 77.456 82.535845) (end 76.814155 81.894) (width 0.25) (layer "F.Cu") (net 12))
 (segment (start 76.814155 81.894) (end 75.329449 81.894) (width 0.25) (layer "F.Cu") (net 12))
 (segment (start 78.904155 83.984) (end 78.055845 83.984) (width 0.25) (layer "F.Cu") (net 12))
 (segment (start 87.66 92.739845) (end 78.904155 83.984) (width 0.25) (layer "F.Cu") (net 12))
 (segment (start 86.36 101.52) (end 87.66 100.22) (width 0.25) (layer "F.Cu") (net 12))
 (segment (start 75.329449 81.894) (end 74.016 80.580551) (width 0.25) (layer "F.Cu") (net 12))
 (segment (start 72.149 73.824) (end 77.456 73.824) (width 0.25) (layer "B.Cu") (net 12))
 (segment (start 77.456 73.824) (end 78.48 72.8) (width 0.25) (layer "B.Cu") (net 12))
 (segment (start 71.125 72.8) (end 72.149 73.824) (width 0.25) (layer "B.Cu") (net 12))
 (segment (start 74.916 85.302845) (end 71.549155 81.936) (width 0.25) (layer "F.Cu") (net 15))
 (segment (start 70.101 81.936) (end 68.585 80.42) (width 0.25) (layer "F.Cu") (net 15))
 (segment (start 86.36 106.52) (end 85.586 107.294) (width 0.25) (layer "F.Cu") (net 15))
 (segment (start 74.916 106.244155) (end 74.916 85.302845) (width 0.25) (layer "F.Cu") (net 15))
 (segment (start 71.549155 81.936) (end 70.101 81.936) (width 0.25) (layer "F.Cu") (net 15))
 (segment (start 85.586 107.294) (end 75.965845 107.294) (width 0.25) (layer "F.Cu") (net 15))
 (segment (start 75.965845 107.294) (end 74.916 106.244155) (width 0.25) (layer "F.Cu") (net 15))
 (segment (start 75.94 80.42) (end 74.916 79.396) (width 0.25) (layer "B.Cu") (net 15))
 (segment (start 69.609 79.396) (end 68.585 80.42) (width 0.25) (layer "B.Cu") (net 15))
 (segment (start 74.916 79.396) (end 69.609 79.396) (width 0.25) (layer "B.Cu") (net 15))
 (segment (start 86.36 96.52) (end 82.7 96.52) (width 0.25) (layer "F.Cu") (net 32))
 (segment (start 82.7 96.52) (end 78.48 100.74) (width 0.25) (layer "F.Cu") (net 32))
 (segment (start 71.125 100.74) (end 72.149 101.764) (width 0.25) (layer "B.Cu") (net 32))
 (segment (start 72.149 101.764) (end 77.456 101.764) (width 0.25) (layer "B.Cu") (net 32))
 (segment (start 77.456 101.764) (end 78.48 100.74) (width 0.25) (layer "B.Cu") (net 32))
 (segment (start 85.28 99.02) (end 78.48 105.82) (width 0.25) (layer "F.Cu") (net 36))
 (segment (start 86.36 99.02) (end 85.28 99.02) (width 0.25) (layer "F.Cu") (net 36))
 (segment (start 71.125 105.82) (end 72.149 106.844) (width 0.25) (layer "B.Cu") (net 36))
 (segment (start 77.456 106.844) (end 78.48 105.82) (width 0.25) (layer "B.Cu") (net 36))
 (segment (start 72.149 106.844) (end 77.456 106.844) (width 0.25) (layer "B.Cu") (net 36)))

